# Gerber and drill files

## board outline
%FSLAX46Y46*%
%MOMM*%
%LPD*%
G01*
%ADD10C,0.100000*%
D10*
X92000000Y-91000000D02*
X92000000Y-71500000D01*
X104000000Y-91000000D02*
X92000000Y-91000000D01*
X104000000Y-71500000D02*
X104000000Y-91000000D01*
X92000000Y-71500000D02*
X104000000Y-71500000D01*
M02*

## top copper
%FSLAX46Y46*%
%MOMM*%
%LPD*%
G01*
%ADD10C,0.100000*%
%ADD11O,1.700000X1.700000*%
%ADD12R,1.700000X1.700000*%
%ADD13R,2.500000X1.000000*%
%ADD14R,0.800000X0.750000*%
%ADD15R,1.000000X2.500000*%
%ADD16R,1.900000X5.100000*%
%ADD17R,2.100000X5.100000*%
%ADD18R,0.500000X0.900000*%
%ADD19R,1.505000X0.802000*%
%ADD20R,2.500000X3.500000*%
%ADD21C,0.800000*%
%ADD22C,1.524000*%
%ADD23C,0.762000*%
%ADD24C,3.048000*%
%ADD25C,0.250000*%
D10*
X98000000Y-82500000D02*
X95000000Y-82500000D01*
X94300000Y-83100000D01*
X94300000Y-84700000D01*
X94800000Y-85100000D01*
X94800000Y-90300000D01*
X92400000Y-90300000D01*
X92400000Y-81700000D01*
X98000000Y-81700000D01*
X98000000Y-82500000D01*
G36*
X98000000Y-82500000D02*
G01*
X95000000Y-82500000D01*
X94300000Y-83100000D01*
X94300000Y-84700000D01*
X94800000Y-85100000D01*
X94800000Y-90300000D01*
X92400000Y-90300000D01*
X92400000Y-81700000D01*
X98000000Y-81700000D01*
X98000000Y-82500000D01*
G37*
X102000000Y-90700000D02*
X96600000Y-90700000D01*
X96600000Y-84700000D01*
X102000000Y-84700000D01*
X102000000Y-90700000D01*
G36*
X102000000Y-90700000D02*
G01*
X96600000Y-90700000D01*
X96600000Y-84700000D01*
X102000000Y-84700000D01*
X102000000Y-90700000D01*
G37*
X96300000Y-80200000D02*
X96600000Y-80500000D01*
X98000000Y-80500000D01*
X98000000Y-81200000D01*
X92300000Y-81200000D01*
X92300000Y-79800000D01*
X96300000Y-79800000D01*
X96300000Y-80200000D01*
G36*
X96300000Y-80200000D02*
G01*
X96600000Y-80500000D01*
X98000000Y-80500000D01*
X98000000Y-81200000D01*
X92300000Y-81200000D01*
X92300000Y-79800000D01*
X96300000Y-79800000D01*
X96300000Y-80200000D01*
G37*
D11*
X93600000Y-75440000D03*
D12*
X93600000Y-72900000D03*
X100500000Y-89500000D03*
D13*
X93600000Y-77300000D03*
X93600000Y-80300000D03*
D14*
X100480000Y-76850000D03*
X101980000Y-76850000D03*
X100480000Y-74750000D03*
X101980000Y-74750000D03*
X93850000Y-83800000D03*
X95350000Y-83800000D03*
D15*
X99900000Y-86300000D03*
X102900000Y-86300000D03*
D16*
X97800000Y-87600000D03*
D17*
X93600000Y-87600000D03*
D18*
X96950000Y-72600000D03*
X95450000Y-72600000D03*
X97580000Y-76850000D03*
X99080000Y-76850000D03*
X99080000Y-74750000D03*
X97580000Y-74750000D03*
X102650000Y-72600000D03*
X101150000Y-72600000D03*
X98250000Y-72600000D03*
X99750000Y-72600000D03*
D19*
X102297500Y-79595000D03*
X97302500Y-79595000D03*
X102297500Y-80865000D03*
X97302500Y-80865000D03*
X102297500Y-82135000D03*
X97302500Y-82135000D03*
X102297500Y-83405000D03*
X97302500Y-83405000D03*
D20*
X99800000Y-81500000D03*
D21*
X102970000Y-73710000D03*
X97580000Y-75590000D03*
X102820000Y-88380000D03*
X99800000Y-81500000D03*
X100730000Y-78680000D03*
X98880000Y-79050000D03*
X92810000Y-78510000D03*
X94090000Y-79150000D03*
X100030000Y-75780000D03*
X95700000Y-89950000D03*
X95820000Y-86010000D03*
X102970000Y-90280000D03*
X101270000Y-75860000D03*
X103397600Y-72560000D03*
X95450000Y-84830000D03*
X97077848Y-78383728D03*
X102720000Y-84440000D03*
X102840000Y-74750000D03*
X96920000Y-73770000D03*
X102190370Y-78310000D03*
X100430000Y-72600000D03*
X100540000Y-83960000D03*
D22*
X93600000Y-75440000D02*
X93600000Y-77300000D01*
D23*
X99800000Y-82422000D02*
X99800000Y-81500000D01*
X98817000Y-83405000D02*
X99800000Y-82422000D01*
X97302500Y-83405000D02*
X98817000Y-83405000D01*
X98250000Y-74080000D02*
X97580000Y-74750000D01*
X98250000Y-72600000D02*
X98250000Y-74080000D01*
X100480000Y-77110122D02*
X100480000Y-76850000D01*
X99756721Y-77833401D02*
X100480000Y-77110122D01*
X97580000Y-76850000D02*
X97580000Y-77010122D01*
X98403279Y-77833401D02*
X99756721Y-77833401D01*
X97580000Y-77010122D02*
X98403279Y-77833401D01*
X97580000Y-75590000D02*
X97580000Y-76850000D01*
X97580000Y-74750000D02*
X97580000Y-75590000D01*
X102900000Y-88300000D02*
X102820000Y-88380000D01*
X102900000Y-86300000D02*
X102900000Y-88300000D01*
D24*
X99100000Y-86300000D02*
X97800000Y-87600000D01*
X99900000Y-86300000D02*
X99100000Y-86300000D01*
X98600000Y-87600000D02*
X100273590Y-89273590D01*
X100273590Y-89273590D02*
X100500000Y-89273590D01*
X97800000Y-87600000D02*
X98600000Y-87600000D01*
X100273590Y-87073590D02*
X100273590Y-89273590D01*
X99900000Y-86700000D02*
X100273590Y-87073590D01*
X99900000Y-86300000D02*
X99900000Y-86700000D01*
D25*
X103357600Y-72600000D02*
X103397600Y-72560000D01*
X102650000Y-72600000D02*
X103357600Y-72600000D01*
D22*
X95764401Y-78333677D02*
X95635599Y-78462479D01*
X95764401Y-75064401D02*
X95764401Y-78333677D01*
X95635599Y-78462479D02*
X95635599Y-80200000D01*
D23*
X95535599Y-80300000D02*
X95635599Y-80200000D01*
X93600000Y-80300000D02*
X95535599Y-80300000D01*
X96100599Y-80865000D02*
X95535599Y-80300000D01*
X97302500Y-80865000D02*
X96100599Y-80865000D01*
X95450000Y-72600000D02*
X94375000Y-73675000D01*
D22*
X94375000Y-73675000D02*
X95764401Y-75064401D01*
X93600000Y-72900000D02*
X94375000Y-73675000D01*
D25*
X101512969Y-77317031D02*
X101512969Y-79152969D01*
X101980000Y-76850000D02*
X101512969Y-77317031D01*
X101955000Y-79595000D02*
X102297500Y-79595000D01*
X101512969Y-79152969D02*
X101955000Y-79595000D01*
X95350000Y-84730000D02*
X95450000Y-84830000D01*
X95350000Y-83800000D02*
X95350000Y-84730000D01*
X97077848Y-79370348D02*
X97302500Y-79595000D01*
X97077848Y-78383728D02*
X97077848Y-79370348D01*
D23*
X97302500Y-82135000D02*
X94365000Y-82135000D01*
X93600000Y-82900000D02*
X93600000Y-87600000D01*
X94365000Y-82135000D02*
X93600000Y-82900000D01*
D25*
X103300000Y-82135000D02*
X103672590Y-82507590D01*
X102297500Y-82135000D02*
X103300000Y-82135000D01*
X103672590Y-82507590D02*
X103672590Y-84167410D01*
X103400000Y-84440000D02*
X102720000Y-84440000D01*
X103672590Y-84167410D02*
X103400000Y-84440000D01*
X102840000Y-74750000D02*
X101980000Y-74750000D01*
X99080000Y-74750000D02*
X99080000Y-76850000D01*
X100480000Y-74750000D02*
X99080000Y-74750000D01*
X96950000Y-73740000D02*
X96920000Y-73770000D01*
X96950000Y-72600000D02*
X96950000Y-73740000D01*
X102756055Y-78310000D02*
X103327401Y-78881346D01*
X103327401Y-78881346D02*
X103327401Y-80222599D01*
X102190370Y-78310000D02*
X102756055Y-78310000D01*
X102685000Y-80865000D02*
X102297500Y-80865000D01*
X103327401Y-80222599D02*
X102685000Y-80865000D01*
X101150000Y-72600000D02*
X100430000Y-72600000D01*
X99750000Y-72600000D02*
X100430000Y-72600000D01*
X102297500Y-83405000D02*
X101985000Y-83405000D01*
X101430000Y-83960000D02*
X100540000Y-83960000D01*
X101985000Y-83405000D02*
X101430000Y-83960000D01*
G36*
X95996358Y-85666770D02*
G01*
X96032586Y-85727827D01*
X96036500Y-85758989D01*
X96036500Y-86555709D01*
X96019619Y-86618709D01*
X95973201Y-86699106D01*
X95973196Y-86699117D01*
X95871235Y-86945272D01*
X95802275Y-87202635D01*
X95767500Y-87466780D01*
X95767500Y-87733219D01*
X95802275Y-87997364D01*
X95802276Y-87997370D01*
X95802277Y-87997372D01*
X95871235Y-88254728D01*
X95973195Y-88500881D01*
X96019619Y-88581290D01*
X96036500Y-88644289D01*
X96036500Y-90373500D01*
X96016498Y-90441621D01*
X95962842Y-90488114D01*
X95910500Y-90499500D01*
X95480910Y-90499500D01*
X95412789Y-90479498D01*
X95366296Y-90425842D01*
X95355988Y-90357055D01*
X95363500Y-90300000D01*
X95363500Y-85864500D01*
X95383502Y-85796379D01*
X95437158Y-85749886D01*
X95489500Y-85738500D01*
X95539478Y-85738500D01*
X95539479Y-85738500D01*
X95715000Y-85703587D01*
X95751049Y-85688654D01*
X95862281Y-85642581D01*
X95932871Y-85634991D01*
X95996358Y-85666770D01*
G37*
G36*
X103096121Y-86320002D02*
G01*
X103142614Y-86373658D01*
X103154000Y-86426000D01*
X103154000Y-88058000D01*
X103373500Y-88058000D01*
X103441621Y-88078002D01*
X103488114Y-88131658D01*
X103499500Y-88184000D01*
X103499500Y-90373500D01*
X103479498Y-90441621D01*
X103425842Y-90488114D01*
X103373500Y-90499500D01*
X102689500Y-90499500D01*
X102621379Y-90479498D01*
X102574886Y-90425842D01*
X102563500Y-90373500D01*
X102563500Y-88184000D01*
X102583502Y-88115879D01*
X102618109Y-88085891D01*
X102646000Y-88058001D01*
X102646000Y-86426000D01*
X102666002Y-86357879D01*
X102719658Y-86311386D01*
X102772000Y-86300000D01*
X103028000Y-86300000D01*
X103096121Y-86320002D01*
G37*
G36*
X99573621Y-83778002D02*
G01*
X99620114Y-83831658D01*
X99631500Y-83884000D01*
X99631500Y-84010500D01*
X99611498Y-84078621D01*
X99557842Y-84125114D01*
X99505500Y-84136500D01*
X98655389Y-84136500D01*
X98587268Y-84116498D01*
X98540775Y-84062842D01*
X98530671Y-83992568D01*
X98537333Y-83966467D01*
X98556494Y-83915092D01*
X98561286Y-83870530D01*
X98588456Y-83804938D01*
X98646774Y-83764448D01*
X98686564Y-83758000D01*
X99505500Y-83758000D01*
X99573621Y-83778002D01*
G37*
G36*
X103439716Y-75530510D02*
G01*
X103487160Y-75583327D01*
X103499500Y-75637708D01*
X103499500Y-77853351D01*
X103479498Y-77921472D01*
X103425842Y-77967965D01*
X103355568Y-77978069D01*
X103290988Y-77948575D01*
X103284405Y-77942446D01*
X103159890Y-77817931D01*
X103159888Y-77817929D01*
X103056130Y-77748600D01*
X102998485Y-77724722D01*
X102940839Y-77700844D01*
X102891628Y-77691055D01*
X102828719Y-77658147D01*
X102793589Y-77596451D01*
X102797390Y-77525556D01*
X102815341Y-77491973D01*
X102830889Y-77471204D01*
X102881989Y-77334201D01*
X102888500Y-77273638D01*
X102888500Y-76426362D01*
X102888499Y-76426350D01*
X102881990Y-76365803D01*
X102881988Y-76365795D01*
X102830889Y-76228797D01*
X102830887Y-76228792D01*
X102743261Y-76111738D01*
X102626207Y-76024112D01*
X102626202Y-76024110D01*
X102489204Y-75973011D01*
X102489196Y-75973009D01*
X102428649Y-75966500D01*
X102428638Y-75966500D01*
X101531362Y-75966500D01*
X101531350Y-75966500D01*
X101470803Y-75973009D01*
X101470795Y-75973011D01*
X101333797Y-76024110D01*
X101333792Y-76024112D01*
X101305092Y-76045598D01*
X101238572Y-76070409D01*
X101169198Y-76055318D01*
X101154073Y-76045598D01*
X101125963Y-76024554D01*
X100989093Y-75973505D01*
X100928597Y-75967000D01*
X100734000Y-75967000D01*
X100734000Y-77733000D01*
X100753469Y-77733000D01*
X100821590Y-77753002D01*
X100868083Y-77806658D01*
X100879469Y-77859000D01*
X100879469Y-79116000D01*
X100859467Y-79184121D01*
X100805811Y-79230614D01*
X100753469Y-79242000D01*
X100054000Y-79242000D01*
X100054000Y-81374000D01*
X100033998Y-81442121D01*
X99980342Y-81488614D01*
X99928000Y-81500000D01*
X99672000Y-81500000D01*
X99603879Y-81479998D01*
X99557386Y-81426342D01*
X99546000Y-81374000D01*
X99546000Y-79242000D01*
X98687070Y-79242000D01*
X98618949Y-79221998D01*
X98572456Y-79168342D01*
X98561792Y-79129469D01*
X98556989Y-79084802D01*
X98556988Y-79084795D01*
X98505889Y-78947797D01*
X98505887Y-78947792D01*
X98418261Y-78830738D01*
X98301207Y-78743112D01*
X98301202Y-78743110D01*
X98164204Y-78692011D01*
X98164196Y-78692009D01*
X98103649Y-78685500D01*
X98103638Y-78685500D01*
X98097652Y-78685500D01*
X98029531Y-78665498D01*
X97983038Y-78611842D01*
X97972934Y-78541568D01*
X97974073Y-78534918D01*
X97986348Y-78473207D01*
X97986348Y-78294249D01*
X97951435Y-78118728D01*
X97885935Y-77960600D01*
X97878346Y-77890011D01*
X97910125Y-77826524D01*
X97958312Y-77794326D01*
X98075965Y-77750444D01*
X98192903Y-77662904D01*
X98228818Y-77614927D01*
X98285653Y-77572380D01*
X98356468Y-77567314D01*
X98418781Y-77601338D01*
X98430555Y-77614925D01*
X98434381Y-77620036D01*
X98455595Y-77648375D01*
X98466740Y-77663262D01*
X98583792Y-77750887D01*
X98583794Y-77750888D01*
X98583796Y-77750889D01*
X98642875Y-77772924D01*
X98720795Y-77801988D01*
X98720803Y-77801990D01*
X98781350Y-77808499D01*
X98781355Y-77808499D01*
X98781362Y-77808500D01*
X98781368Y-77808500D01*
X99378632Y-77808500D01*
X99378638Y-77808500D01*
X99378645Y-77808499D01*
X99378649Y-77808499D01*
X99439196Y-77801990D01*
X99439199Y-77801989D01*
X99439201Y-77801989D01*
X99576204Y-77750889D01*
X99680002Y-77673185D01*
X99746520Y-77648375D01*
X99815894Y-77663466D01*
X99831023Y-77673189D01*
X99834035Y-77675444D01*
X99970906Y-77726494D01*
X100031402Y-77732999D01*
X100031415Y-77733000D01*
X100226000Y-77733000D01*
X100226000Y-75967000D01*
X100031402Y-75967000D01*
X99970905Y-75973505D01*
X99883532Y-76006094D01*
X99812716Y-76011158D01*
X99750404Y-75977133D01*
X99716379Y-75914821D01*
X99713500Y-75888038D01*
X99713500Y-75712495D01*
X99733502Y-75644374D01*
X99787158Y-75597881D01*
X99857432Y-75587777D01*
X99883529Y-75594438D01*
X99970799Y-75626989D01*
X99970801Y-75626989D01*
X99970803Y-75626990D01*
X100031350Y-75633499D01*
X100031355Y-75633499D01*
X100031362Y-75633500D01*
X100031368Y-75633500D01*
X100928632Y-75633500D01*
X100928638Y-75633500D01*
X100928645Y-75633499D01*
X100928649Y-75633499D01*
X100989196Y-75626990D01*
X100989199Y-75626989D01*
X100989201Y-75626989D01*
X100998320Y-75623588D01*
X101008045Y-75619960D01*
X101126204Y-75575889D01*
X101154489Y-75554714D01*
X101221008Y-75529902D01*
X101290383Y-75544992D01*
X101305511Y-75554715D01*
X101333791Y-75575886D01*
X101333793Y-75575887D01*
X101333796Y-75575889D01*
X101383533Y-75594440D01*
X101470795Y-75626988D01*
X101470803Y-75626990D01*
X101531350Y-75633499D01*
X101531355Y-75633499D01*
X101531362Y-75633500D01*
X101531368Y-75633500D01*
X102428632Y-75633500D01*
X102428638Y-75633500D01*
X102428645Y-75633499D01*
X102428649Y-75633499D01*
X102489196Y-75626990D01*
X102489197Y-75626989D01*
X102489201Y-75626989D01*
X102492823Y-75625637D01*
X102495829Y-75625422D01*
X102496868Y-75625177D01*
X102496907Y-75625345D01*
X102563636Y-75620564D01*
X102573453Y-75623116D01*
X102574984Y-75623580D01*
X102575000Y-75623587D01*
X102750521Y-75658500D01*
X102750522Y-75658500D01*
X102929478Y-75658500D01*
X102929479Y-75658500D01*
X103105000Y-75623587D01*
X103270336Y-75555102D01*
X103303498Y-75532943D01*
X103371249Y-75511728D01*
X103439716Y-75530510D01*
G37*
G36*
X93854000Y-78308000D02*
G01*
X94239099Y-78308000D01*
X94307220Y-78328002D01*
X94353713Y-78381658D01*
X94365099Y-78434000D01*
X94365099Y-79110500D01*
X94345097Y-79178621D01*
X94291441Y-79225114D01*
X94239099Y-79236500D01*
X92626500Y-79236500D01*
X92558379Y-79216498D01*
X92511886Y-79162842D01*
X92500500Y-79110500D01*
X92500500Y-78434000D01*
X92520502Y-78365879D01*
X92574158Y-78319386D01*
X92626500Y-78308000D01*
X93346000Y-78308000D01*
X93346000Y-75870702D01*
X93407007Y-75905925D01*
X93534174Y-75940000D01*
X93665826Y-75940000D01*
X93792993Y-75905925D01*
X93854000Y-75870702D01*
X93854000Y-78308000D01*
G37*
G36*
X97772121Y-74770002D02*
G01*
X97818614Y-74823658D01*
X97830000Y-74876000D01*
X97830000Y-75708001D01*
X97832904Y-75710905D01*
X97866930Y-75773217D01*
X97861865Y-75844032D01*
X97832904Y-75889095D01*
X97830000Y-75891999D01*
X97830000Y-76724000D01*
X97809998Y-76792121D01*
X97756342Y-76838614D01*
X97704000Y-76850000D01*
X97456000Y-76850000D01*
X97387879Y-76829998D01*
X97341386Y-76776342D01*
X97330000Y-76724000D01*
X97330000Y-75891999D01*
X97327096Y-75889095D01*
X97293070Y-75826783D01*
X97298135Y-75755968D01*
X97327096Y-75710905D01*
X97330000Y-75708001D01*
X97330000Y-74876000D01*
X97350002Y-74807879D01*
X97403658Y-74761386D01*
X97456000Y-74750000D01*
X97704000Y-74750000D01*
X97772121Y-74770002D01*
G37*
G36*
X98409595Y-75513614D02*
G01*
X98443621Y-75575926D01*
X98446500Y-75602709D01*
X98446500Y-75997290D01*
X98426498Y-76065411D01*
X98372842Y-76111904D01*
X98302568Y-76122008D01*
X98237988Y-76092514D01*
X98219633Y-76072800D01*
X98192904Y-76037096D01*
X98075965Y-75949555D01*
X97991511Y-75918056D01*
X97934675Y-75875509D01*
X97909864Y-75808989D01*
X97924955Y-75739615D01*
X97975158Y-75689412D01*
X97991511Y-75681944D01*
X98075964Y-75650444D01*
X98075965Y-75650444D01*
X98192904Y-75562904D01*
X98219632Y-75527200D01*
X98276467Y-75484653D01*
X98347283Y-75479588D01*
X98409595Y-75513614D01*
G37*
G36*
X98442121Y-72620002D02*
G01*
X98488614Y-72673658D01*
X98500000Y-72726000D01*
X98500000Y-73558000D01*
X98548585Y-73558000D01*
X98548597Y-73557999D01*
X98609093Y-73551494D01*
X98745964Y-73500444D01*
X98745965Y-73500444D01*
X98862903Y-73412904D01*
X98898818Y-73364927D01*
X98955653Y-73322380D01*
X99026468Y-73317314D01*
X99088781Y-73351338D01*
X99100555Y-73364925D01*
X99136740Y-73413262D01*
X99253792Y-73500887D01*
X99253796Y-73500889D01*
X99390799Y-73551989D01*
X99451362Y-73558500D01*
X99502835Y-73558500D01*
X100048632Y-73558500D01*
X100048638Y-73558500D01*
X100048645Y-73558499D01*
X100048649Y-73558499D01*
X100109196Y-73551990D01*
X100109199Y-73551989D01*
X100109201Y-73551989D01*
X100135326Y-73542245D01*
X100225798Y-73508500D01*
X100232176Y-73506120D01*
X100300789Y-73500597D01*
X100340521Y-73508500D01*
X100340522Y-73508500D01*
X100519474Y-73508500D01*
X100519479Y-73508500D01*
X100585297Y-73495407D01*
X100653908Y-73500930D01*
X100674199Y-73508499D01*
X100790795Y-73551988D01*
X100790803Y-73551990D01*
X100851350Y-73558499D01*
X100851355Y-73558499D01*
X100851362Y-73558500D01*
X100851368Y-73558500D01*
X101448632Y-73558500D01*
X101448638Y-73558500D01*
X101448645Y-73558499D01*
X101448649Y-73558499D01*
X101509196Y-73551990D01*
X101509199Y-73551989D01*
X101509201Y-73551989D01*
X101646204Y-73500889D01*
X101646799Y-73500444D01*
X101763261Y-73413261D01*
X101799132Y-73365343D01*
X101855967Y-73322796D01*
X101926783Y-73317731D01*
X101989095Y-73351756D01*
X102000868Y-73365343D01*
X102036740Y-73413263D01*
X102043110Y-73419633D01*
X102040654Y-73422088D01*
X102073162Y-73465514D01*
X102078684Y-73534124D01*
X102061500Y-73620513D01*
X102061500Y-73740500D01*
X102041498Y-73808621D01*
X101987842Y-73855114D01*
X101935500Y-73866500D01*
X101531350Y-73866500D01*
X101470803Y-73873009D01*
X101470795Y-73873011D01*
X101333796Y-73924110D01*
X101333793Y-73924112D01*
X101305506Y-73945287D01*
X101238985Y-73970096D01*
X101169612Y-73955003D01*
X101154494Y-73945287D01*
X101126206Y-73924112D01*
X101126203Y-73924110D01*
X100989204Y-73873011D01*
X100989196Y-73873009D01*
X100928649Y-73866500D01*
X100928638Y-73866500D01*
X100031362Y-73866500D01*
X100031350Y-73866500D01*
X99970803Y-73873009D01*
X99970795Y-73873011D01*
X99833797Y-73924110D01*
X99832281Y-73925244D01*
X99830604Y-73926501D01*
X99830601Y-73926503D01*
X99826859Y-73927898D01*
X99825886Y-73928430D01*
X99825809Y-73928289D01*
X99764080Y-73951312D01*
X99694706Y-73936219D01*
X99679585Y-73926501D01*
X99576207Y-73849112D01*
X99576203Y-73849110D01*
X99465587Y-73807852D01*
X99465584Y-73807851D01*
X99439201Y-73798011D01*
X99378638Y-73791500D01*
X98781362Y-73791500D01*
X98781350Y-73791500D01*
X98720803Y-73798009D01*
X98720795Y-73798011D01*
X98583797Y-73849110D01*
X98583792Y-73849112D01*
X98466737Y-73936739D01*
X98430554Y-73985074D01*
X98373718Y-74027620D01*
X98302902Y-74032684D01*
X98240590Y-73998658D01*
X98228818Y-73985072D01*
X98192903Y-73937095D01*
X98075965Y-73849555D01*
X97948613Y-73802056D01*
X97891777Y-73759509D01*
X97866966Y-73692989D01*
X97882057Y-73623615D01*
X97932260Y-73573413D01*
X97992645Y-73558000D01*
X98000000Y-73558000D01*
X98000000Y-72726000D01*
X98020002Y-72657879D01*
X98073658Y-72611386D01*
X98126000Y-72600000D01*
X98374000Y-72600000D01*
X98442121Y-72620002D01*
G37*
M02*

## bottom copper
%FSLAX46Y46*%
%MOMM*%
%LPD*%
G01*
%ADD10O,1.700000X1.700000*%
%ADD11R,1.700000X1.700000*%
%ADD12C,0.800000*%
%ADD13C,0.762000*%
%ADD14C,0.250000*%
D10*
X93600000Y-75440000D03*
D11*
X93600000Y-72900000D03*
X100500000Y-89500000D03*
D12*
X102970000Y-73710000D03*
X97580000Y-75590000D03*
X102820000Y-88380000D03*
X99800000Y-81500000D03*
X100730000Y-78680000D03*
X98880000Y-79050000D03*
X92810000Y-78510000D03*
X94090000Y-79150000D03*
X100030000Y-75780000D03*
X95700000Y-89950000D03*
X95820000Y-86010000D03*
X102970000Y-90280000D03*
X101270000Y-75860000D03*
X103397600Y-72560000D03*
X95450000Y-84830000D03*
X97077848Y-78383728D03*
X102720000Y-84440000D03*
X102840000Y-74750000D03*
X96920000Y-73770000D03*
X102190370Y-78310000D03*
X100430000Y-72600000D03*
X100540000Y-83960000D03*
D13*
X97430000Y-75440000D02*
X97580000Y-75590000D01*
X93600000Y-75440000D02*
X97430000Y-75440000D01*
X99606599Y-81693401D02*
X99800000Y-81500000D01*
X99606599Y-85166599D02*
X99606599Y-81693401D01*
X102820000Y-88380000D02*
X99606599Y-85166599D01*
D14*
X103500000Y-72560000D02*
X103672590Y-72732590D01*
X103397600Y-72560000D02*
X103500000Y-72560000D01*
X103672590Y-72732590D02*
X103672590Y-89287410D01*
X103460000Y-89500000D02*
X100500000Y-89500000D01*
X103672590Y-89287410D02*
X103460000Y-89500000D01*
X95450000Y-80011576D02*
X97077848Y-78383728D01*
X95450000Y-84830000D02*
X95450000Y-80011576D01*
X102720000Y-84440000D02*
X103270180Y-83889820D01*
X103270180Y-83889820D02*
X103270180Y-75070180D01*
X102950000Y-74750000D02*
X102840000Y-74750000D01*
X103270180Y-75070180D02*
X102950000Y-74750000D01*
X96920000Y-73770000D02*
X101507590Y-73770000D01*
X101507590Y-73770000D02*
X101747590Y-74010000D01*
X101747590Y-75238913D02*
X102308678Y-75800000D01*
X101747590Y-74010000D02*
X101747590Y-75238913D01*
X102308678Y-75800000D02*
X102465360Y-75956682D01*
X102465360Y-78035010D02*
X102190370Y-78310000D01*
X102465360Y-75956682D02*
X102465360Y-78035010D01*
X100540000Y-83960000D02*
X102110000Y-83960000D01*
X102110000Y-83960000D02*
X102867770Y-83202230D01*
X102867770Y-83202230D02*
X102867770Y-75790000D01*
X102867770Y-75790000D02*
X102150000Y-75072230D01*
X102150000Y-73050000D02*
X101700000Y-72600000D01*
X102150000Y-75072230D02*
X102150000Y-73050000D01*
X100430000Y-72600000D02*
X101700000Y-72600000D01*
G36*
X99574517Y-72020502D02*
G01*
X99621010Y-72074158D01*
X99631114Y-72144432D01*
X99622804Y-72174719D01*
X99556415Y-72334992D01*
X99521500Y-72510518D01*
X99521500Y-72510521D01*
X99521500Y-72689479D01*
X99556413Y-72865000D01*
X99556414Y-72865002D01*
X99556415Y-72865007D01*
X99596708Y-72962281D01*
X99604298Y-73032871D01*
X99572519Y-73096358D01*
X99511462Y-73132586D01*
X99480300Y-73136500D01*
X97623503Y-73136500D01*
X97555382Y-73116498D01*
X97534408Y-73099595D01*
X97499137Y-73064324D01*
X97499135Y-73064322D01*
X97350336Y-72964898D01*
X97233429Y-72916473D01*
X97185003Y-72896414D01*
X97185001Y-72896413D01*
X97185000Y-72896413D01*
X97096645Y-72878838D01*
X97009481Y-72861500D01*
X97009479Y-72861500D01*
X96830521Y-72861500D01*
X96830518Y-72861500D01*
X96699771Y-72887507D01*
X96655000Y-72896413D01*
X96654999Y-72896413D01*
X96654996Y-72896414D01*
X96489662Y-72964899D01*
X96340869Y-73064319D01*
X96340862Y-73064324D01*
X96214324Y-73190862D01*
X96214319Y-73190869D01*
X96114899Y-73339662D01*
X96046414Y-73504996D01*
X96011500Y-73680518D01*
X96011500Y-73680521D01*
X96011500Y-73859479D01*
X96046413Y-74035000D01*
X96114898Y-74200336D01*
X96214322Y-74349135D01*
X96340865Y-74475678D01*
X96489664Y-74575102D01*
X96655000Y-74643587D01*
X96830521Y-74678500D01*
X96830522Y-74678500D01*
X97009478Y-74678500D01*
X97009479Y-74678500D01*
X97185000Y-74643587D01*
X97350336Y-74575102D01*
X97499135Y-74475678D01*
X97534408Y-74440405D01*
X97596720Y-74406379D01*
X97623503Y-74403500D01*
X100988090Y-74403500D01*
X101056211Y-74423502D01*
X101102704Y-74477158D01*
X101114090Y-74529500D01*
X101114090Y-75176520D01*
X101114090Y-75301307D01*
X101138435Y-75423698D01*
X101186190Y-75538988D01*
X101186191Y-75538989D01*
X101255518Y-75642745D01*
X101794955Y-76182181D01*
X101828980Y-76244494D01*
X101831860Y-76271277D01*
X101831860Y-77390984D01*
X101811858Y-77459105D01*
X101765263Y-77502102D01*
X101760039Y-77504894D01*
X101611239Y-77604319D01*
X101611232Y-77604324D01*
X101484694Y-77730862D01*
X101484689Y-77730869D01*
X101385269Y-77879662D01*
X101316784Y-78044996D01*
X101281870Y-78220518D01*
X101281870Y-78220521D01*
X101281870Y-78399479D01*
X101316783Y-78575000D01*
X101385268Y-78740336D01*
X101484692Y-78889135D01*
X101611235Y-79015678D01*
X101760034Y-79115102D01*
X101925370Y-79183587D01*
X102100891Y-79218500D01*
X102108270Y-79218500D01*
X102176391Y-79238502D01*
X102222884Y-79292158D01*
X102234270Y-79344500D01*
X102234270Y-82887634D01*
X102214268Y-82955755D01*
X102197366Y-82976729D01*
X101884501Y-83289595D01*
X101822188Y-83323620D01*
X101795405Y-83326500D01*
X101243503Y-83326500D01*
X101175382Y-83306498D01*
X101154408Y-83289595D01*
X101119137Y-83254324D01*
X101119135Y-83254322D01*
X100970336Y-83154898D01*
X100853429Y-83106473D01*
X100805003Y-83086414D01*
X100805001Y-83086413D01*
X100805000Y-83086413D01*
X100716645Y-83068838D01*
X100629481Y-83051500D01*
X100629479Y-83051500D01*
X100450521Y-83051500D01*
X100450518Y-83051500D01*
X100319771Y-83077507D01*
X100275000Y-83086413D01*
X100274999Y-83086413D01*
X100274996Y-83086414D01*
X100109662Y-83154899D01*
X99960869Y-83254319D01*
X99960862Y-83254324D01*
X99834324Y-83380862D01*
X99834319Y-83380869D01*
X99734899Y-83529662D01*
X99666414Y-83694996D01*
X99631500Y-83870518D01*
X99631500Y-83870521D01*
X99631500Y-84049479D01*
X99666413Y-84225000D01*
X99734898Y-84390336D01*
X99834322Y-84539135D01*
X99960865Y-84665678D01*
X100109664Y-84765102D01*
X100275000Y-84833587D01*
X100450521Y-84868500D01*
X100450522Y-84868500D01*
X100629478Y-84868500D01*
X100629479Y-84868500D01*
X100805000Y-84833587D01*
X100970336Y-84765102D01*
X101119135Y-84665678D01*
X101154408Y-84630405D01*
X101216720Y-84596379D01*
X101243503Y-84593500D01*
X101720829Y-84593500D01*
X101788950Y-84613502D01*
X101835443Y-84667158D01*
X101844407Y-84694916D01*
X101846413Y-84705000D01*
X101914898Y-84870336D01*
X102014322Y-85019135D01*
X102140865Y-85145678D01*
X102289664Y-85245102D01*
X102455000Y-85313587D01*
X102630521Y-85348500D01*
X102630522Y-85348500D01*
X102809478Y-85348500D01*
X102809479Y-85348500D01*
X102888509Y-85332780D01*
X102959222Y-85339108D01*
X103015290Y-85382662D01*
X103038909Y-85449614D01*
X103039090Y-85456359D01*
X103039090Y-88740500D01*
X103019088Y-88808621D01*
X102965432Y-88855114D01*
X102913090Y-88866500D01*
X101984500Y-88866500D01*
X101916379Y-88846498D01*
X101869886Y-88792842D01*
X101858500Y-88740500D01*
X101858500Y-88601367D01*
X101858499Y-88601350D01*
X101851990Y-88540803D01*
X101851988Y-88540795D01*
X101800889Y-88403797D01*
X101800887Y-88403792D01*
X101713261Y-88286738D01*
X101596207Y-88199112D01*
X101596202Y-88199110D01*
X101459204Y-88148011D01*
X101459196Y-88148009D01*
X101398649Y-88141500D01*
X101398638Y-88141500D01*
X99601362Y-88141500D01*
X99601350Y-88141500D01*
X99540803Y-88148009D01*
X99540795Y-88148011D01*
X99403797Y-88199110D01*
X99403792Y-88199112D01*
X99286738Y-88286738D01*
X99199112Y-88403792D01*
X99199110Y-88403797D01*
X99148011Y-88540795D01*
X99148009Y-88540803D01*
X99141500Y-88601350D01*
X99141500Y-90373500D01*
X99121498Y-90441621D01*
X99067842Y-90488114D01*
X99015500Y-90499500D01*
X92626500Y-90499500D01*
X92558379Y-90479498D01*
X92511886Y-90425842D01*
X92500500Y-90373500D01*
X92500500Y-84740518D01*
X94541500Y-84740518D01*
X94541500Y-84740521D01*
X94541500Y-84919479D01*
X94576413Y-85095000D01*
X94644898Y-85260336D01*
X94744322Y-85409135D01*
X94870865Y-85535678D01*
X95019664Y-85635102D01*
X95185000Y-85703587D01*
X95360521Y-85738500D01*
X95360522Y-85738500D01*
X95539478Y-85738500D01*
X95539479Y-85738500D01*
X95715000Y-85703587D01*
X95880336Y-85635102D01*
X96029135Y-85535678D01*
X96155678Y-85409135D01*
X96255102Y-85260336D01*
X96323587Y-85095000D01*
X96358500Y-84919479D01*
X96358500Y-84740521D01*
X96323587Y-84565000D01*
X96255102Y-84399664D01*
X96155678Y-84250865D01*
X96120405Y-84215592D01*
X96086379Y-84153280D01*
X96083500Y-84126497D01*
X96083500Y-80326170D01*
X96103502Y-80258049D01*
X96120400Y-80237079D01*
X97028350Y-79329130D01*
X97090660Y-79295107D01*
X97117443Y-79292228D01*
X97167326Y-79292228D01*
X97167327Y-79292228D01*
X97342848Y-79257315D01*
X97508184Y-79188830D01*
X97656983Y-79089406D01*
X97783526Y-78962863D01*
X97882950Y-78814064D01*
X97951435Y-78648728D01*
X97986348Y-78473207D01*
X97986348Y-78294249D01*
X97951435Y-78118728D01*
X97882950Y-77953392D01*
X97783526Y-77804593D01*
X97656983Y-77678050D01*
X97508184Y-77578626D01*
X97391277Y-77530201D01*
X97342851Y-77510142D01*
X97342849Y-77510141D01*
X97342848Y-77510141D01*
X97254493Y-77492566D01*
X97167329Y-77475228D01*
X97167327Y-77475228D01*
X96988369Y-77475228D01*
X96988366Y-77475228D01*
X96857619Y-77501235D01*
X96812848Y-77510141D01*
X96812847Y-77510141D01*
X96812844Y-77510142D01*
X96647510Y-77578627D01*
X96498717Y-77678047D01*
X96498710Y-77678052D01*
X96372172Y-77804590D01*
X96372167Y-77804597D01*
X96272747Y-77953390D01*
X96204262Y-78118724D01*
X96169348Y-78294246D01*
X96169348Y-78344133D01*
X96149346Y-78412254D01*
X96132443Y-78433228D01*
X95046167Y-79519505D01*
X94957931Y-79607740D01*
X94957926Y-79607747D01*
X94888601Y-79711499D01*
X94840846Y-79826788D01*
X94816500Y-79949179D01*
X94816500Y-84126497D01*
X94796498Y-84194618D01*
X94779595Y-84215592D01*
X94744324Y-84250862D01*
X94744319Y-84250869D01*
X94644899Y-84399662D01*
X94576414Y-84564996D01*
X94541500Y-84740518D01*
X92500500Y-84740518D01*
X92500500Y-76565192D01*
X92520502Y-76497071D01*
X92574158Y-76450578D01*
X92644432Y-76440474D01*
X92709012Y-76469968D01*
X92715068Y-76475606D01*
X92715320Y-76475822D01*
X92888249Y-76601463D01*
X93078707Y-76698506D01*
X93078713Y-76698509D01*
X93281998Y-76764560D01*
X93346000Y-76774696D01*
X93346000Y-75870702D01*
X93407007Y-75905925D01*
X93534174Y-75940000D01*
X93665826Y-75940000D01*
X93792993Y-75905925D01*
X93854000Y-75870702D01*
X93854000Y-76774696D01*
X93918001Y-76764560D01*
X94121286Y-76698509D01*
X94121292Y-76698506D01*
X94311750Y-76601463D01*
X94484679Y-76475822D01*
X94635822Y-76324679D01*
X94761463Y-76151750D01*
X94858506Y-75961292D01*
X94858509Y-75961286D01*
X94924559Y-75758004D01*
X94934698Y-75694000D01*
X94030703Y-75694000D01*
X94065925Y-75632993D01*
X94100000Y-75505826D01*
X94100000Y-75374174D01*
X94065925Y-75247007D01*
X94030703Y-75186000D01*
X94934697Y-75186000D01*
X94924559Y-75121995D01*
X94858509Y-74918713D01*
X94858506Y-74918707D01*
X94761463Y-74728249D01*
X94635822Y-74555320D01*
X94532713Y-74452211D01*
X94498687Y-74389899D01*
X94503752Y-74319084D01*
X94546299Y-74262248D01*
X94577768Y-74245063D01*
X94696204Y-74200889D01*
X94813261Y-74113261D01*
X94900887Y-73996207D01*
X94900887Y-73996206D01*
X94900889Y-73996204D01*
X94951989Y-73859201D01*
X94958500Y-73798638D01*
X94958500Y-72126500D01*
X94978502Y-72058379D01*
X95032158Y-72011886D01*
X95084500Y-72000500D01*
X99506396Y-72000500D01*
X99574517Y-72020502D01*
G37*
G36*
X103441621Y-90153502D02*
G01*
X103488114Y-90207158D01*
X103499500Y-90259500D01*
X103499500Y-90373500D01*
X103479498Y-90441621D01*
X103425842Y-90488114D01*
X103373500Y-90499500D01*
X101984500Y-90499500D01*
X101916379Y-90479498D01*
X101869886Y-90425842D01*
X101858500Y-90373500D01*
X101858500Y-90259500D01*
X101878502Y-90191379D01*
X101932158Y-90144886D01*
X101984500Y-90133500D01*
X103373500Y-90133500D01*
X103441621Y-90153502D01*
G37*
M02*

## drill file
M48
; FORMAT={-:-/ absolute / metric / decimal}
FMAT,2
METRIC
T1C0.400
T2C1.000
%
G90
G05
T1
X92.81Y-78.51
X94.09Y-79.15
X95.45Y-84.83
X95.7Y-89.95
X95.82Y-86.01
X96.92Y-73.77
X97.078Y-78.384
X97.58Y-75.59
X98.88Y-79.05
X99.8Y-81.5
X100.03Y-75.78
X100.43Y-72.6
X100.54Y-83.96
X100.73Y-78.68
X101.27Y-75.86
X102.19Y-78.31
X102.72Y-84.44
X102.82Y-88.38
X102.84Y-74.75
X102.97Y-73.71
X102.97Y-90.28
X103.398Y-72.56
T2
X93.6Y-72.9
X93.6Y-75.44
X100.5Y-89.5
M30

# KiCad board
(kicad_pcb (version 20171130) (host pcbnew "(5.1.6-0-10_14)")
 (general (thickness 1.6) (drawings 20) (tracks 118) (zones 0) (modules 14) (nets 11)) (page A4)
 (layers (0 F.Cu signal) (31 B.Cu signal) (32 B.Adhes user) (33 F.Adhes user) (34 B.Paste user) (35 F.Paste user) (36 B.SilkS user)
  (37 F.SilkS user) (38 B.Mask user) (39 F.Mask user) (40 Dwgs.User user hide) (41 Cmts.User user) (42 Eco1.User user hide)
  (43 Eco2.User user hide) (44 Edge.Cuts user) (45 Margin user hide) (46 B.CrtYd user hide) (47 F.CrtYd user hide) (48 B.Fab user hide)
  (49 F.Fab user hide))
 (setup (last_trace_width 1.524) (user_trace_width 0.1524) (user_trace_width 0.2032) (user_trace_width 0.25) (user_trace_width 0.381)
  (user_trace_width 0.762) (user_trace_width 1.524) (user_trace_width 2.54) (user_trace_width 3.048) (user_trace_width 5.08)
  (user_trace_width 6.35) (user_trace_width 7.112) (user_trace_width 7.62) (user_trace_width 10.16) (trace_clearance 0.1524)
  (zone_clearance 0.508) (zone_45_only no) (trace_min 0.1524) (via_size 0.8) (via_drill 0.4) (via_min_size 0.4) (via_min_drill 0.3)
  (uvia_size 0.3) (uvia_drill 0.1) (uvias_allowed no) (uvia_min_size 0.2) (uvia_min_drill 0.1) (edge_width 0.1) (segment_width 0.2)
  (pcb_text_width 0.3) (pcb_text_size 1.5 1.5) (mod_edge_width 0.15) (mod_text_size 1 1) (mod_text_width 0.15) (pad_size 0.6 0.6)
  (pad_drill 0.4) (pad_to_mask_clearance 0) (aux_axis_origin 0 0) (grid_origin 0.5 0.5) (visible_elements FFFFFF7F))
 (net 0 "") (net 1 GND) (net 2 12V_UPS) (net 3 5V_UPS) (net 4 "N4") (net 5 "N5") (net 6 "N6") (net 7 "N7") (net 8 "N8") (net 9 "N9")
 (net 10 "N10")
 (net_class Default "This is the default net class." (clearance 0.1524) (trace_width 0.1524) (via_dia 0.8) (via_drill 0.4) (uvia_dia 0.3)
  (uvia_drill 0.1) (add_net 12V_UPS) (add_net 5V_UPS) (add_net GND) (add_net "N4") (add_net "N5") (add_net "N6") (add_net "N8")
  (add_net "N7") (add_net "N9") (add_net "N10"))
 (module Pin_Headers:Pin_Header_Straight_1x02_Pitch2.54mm (layer F.Cu) (at 93.6 72.9)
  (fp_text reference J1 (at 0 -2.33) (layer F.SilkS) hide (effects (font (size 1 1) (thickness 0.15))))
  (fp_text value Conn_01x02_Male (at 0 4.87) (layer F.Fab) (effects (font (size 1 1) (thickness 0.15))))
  (pad 2 thru_hole oval (at 0 2.54) (size 1.7 1.7) (drill 1) (layers *.Cu *.Mask) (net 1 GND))
  (pad 1 thru_hole rect (at 0 0) (size 1.7 1.7) (drill 1) (layers *.Cu *.Mask) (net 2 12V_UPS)))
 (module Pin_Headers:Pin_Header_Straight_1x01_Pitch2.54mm (layer F.Cu) (at 100.5 89.5)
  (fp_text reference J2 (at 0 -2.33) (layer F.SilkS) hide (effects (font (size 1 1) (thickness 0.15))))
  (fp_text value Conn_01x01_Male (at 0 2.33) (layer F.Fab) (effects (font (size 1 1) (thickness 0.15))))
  (pad 1 thru_hole rect (at 0 0) (size 1.7 1.7) (drill 1) (layers *.Cu *.Mask) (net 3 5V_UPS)))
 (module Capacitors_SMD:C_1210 (layer F.Cu) (at 93.6 78.8 270)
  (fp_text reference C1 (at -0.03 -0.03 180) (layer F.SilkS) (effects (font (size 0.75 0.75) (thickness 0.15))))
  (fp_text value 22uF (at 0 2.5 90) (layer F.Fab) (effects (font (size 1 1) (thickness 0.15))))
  (pad 1 smd rect (at -1.5 0 270) (size 1 2.5) (layers F.Cu F.Paste F.Mask) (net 1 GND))
  (pad 2 smd rect (at 1.5 0 270) (size 1 2.5) (layers F.Cu F.Paste F.Mask) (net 2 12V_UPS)))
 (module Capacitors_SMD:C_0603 (layer F.Cu) (at 101.23 76.85)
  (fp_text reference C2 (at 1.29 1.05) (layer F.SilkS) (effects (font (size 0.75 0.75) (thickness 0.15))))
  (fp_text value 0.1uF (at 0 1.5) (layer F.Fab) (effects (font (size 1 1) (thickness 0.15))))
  (pad 1 smd rect (at -0.75 0) (size 0.8 0.75) (layers F.Cu F.Paste F.Mask) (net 1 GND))
  (pad 2 smd rect (at 0.75 0) (size 0.8 0.75) (layers F.Cu F.Paste F.Mask) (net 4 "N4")))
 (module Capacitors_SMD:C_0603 (layer F.Cu) (at 101.23 74.75)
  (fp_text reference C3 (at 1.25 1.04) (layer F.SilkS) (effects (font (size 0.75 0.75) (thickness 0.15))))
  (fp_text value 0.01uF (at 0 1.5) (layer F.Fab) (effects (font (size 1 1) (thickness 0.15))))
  (pad 1 smd rect (at -0.75 0) (size 0.8 0.75) (layers F.Cu F.Paste F.Mask) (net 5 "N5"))
  (pad 2 smd rect (at 0.75 0) (size 0.8 0.75) (layers F.Cu F.Paste F.Mask) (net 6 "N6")))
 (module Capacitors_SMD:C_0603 (layer F.Cu) (at 94.6 83.8 180)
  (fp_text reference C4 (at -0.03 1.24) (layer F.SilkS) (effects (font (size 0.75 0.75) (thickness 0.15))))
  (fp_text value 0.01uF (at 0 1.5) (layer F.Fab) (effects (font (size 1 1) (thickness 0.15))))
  (pad 2 smd rect (at 0.75 0 180) (size 0.8 0.75) (layers F.Cu F.Paste F.Mask) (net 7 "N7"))
  (pad 1 smd rect (at -0.75 0 180) (size 0.8 0.75) (layers F.Cu F.Paste F.Mask) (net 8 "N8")))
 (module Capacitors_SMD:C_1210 (layer F.Cu) (at 101.4 86.3 180)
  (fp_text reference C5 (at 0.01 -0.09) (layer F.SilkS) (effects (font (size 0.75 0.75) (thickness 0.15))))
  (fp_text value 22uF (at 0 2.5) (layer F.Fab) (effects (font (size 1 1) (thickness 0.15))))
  (pad 2 smd rect (at 1.5 0 180) (size 1 2.5) (layers F.Cu F.Paste F.Mask) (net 3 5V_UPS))
  (pad 1 smd rect (at -1.5 0 180) (size 1 2.5) (layers F.Cu F.Paste F.Mask) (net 1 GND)))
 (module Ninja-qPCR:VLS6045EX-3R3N (layer F.Cu) (at 95.7 87.6 180)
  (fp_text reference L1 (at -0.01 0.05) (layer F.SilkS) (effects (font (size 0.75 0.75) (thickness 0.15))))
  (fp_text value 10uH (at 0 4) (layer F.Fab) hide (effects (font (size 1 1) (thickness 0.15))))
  (pad 1 smd rect (at -2.1 0 180) (size 1.9 5.1) (layers F.Cu F.Paste F.Mask) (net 3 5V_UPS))
  (pad 2 smd rect (at 2.1 0 180) (size 2.1 5.1) (layers F.Cu F.Paste F.Mask) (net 7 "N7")))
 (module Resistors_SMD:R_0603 (layer F.Cu) (at 96.2 72.6)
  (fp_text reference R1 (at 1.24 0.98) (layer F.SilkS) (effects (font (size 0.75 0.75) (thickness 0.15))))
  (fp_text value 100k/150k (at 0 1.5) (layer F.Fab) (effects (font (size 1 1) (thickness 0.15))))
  (pad 2 smd rect (at 0.75 0) (size 0.5 0.9) (layers F.Cu F.Paste F.Mask) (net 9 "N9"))
  (pad 1 smd rect (at -0.75 0) (size 0.5 0.9) (layers F.Cu F.Paste F.Mask) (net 2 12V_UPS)))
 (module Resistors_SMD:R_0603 (layer F.Cu) (at 98.33 76.85 180)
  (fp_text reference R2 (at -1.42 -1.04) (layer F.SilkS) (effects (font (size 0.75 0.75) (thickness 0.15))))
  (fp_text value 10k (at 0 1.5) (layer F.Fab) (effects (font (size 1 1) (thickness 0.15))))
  (pad 2 smd rect (at 0.75 0 180) (size 0.5 0.9) (layers F.Cu F.Paste F.Mask) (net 1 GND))
  (pad 1 smd rect (at -0.75 0 180) (size 0.5 0.9) (layers F.Cu F.Paste F.Mask) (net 5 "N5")))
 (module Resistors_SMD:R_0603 (layer F.Cu) (at 98.33 74.75 180)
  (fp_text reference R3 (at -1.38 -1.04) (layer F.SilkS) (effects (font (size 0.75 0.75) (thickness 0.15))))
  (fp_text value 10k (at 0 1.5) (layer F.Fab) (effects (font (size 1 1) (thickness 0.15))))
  (pad 1 smd rect (at -0.75 0 180) (size 0.5 0.9) (layers F.Cu F.Paste F.Mask) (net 5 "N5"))
  (pad 2 smd rect (at 0.75 0 180) (size 0.5 0.9) (layers F.Cu F.Paste F.Mask) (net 1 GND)))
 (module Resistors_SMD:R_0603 (layer F.Cu) (at 101.9 72.6 180)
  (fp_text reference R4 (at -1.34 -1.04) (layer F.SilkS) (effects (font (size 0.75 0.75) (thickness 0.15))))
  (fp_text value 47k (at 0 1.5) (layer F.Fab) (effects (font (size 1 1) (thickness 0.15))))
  (pad 1 smd rect (at -0.75 0 180) (size 0.5 0.9) (layers F.Cu F.Paste F.Mask) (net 3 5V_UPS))
  (pad 2 smd rect (at 0.75 0 180) (size 0.5 0.9) (layers F.Cu F.Paste F.Mask) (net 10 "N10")))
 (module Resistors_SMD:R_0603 (layer F.Cu) (at 99 72.6 180)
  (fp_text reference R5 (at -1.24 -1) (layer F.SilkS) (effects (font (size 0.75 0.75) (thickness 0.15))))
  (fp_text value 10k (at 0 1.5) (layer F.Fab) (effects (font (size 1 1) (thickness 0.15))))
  (pad 2 smd rect (at 0.75 0 180) (size 0.5 0.9) (layers F.Cu F.Paste F.Mask) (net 1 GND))
  (pad 1 smd rect (at -0.75 0 180) (size 0.5 0.9) (layers F.Cu F.Paste F.Mask) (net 10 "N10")))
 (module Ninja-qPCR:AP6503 (layer F.Cu) (at 99.8 81.5 270)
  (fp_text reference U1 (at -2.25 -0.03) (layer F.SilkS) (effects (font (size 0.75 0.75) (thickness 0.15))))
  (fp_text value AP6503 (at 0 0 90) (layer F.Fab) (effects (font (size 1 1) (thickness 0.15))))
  (pad 8 smd rect (at -1.905 -2.4975 270) (size 0.802 1.505) (layers F.Cu F.Paste F.Mask) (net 4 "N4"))
  (pad 1 smd rect (at -1.905 2.4975 270) (size 0.802 1.505) (layers F.Cu F.Paste F.Mask) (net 8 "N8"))
  (pad 7 smd rect (at -0.635 -2.4975 270) (size 0.802 1.505) (layers F.Cu F.Paste F.Mask) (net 9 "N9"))
  (pad 2 smd rect (at -0.635 2.4975 270) (size 0.802 1.505) (layers F.Cu F.Paste F.Mask) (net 2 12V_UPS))
  (pad 6 smd rect (at 0.635 -2.4975 270) (size 0.802 1.505) (layers F.Cu F.Paste F.Mask) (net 6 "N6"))
  (pad 3 smd rect (at 0.635 2.4975 270) (size 0.802 1.505) (layers F.Cu F.Paste F.Mask) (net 7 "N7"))
  (pad 5 smd rect (at 1.905 -2.4975 270) (size 0.802 1.505) (layers F.Cu F.Paste F.Mask) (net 10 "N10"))
  (pad 4 smd rect (at 1.905 2.4975 270) (size 0.802 1.505) (layers F.Cu F.Paste F.Mask) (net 1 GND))
  (pad 9 smd rect (at 0 0 270) (size 3.5 2.5) (layers F.Cu F.Paste F.Mask) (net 1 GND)))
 (gr_poly
  (pts (xy 98 82.5) (xy 95 82.5) (xy 94.3 83.1) (xy 94.3 84.7) (xy 94.8 85.1) (xy 94.8 90.3) (xy 92.4 90.3) (xy 92.4 81.7) (xy 98 81.7))
  (layer F.Cu) (width 0.1))
 (gr_poly (pts (xy 102 90.7) (xy 96.6 90.7) (xy 96.6 84.7) (xy 102 84.7)) (layer F.Cu) (width 0.1))
 (gr_poly
  (pts (xy 96.3 80.2) (xy 96.6 80.5) (xy 98 80.5) (xy 98 81.2) (xy 92.3 81.2) (xy 92.3 79.8) (xy 96.3 79.8)) (layer F.Cu) (width 0.1))
 (gr_line (start 92 91) (end 92 71.5) (layer Edge.Cuts) (width 0.1))
 (gr_line (start 104 91) (end 92 91) (layer Edge.Cuts) (width 0.1))
 (gr_line (start 104 71.5) (end 104 91) (layer Edge.Cuts) (width 0.1))
 (gr_line (start 92 71.5) (end 104 71.5) (layer Edge.Cuts) (width 0.1))
 (via (at 102.97 73.71) (size 0.8) (drill 0.4) (layers F.Cu B.Cu) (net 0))
 (segment (start 93.6 75.44) (end 93.6 77.3) (width 1.524) (layer F.Cu) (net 1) (status 30))
 (segment (start 99.8 82.422) (end 99.8 81.5) (width 0.762) (layer F.Cu) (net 1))
 (segment (start 98.817 83.405) (end 99.8 82.422) (width 0.762) (layer F.Cu) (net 1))
 (segment (start 97.3025 83.405) (end 98.817 83.405) (width 0.762) (layer F.Cu) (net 1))
 (segment (start 98.25 74.08) (end 97.58 74.75) (width 0.762) (layer F.Cu) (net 1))
 (segment (start 98.25 72.6) (end 98.25 74.08) (width 0.762) (layer F.Cu) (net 1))
 (segment (start 100.48 77.110122) (end 100.48 76.85) (width 0.762) (layer F.Cu) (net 1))
 (segment (start 99.756721 77.833401) (end 100.48 77.110122) (width 0.762) (layer F.Cu) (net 1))
 (segment (start 97.58 76.85) (end 97.58 77.010122) (width 0.762) (layer F.Cu) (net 1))
 (segment (start 98.403279 77.833401) (end 99.756721 77.833401) (width 0.762) (layer F.Cu) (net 1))
 (segment (start 97.58 77.010122) (end 98.403279 77.833401) (width 0.762) (layer F.Cu) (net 1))
 (via (at 97.58 75.59) (size 0.8) (drill 0.4) (layers F.Cu B.Cu) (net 1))
 (segment (start 97.43 75.44) (end 97.58 75.59) (width 0.762) (layer B.Cu) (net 1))
 (segment (start 93.6 75.44) (end 97.43 75.44) (width 0.762) (layer B.Cu) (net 1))
 (segment (start 97.58 75.59) (end 97.58 76.85) (width 0.762) (layer F.Cu) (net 1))
 (segment (start 97.58 74.75) (end 97.58 75.59) (width 0.762) (layer F.Cu) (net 1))
 (segment (start 102.9 88.3) (end 102.82 88.38) (width 0.762) (layer F.Cu) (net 1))
 (via (at 102.82 88.38) (size 0.8) (drill 0.4) (layers F.Cu B.Cu) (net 1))
 (segment (start 102.9 86.3) (end 102.9 88.3) (width 0.762) (layer F.Cu) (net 1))
 (via (at 99.8 81.5) (size 0.8) (drill 0.4) (layers F.Cu B.Cu) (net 1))
 (segment (start 99.606599 81.693401) (end 99.8 81.5) (width 0.762) (layer B.Cu) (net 1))
 (segment (start 99.606599 85.166599) (end 99.606599 81.693401) (width 0.762) (layer B.Cu) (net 1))
 (segment (start 102.82 88.38) (end 99.606599 85.166599) (width 0.762) (layer B.Cu) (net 1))
 (via (at 100.73 78.68) (size 0.8) (drill 0.4) (layers F.Cu B.Cu) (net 1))
 (via (at 98.88 79.05) (size 0.8) (drill 0.4) (layers F.Cu B.Cu) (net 1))
 (via (at 92.81 78.51) (size 0.8) (drill 0.4) (layers F.Cu B.Cu) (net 1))
 (via (at 94.09 79.15) (size 0.8) (drill 0.4) (layers F.Cu B.Cu) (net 1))
 (via (at 100.03 75.78) (size 0.8) (drill 0.4) (layers F.Cu B.Cu) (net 1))
 (via (at 95.7 89.95) (size 0.8) (drill 0.4) (layers F.Cu B.Cu) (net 1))
 (via (at 95.82 86.01) (size 0.8) (drill 0.4) (layers F.Cu B.Cu) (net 1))
 (via (at 102.97 90.28) (size 0.8) (drill 0.4) (layers F.Cu B.Cu) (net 1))
 (via (at 101.27 75.86) (size 0.8) (drill 0.4) (layers F.Cu B.Cu) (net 1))
 (segment (start 99.1 86.3) (end 97.8 87.6) (width 3.048) (layer F.Cu) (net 3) (status 20))
 (segment (start 99.9 86.3) (end 99.1 86.3) (width 3.048) (layer F.Cu) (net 3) (status 10))
 (segment (start 98.6 87.6) (end 100.27359 89.27359) (width 3.048) (layer F.Cu) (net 3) (status 30))
 (segment (start 100.27359 89.27359) (end 100.5 89.27359) (width 3.048) (layer F.Cu) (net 3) (status 30))
 (segment (start 97.8 87.6) (end 98.6 87.6) (width 3.048) (layer F.Cu) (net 3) (status 30))
 (segment (start 100.27359 87.07359) (end 100.27359 89.27359) (width 3.048) (layer F.Cu) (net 3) (status 30))
 (segment (start 99.9 86.7) (end 100.27359 87.07359) (width 3.048) (layer F.Cu) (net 3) (status 30))
 (segment (start 99.9 86.3) (end 99.9 86.7) (width 3.048) (layer F.Cu) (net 3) (status 30))
 (via (at 103.3976 72.56) (size 0.8) (drill 0.4) (layers F.Cu B.Cu) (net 3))
 (segment (start 103.3576 72.6) (end 103.3976 72.56) (width 0.25) (layer F.Cu) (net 3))
 (segment (start 102.65 72.6) (end 103.3576 72.6) (width 0.25) (layer F.Cu) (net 3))
 (segment (start 103.5 72.56) (end 103.67259 72.73259) (width 0.25) (layer B.Cu) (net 3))
 (segment (start 103.3976 72.56) (end 103.5 72.56) (width 0.25) (layer B.Cu) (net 3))
 (segment (start 103.67259 72.73259) (end 103.67259 89.28741) (width 0.25) (layer B.Cu) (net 3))
 (segment (start 103.46 89.5) (end 100.5 89.5) (width 0.25) (layer B.Cu) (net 3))
 (segment (start 103.67259 89.28741) (end 103.46 89.5) (width 0.25) (layer B.Cu) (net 3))
 (segment (start 95.764401 78.333677) (end 95.635599 78.462479) (width 1.524) (layer F.Cu) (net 2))
 (segment (start 95.764401 75.064401) (end 95.764401 78.333677) (width 1.524) (layer F.Cu) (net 2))
 (segment (start 95.635599 78.462479) (end 95.635599 80.2) (width 1.524) (layer F.Cu) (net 2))
 (segment (start 95.535599 80.3) (end 95.635599 80.2) (width 0.762) (layer F.Cu) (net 2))
 (segment (start 93.6 80.3) (end 95.535599 80.3) (width 0.762) (layer F.Cu) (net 2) (status 10))
 (segment (start 96.100599 80.865) (end 95.535599 80.3) (width 0.762) (layer F.Cu) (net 2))
 (segment (start 97.3025 80.865) (end 96.100599 80.865) (width 0.762) (layer F.Cu) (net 2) (status 10))
 (segment (start 95.45 72.6) (end 94.375 73.675) (width 0.762) (layer F.Cu) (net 2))
 (segment (start 94.375 73.675) (end 95.764401 75.064401) (width 1.524) (layer F.Cu) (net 2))
 (segment (start 93.6 72.9) (end 94.375 73.675) (width 1.524) (layer F.Cu) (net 2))
 (segment (start 101.512969 77.317031) (end 101.512969 79.152969) (width 0.25) (layer F.Cu) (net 4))
 (segment (start 101.98 76.85) (end 101.512969 77.317031) (width 0.25) (layer F.Cu) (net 4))
 (segment (start 101.955 79.595) (end 102.2975 79.595) (width 0.25) (layer F.Cu) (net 4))
 (segment (start 101.512969 79.152969) (end 101.955 79.595) (width 0.25) (layer F.Cu) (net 4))
 (via (at 95.45 84.83) (size 0.8) (drill 0.4) (layers F.Cu B.Cu) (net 8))
 (segment (start 95.35 84.73) (end 95.45 84.83) (width 0.25) (layer F.Cu) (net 8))
 (segment (start 95.35 83.8) (end 95.35 84.73) (width 0.25) (layer F.Cu) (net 8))
 (via (at 97.077848 78.383728) (size 0.8) (drill 0.4) (layers F.Cu B.Cu) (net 8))
 (segment (start 95.45 80.011576) (end 97.077848 78.383728) (width 0.25) (layer B.Cu) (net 8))
 (segment (start 95.45 84.83) (end 95.45 80.011576) (width 0.25) (layer B.Cu) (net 8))
 (segment (start 97.077848 79.370348) (end 97.3025 79.595) (width 0.25) (layer F.Cu) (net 8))
 (segment (start 97.077848 78.383728) (end 97.077848 79.370348) (width 0.25) (layer F.Cu) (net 8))
 (segment (start 97.3025 82.135) (end 94.365 82.135) (width 0.762) (layer F.Cu) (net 7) (status 10))
 (segment (start 93.6 82.9) (end 93.6 87.6) (width 0.762) (layer F.Cu) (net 7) (status 20))
 (segment (start 94.365 82.135) (end 93.6 82.9) (width 0.762) (layer F.Cu) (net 7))
 (segment (start 103.3 82.135) (end 103.67259 82.50759) (width 0.25) (layer F.Cu) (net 6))
 (segment (start 102.2975 82.135) (end 103.3 82.135) (width 0.25) (layer F.Cu) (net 6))
 (segment (start 103.67259 82.50759) (end 103.67259 84.16741) (width 0.25) (layer F.Cu) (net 6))
 (via (at 102.72 84.44) (size 0.8) (drill 0.4) (layers F.Cu B.Cu) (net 6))
 (segment (start 103.4 84.44) (end 102.72 84.44) (width 0.25) (layer F.Cu) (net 6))
 (segment (start 103.67259 84.16741) (end 103.4 84.44) (width 0.25) (layer F.Cu) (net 6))
 (segment (start 102.72 84.44) (end 103.27018 83.88982) (width 0.25) (layer B.Cu) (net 6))
 (segment (start 103.27018 83.88982) (end 103.27018 75.07018) (width 0.25) (layer B.Cu) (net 6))
 (via (at 102.84 74.75) (size 0.8) (drill 0.4) (layers F.Cu B.Cu) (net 6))
 (segment (start 102.95 74.75) (end 102.84 74.75) (width 0.25) (layer B.Cu) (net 6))
 (segment (start 103.27018 75.07018) (end 102.95 74.75) (width 0.25) (layer B.Cu) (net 6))
 (segment (start 102.84 74.75) (end 101.98 74.75) (width 0.25) (layer F.Cu) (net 6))
 (segment (start 99.08 74.75) (end 99.08 76.85) (width 0.25) (layer F.Cu) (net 5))
 (segment (start 100.48 74.75) (end 99.08 74.75) (width 0.25) (layer F.Cu) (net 5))
 (via (at 96.92 73.77) (size 0.8) (drill 0.4) (layers F.Cu B.Cu) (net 9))
 (segment (start 96.95 73.74) (end 96.92 73.77) (width 0.25) (layer F.Cu) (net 9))
 (segment (start 96.95 72.6) (end 96.95 73.74) (width 0.25) (layer F.Cu) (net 9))
 (segment (start 96.92 73.77) (end 101.50759 73.77) (width 0.25) (layer B.Cu) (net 9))
 (segment (start 101.50759 73.77) (end 101.74759 74.01) (width 0.25) (layer B.Cu) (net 9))
 (segment (start 101.74759 75.238913) (end 102.308678 75.8) (width 0.25) (layer B.Cu) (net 9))
 (segment (start 101.74759 74.01) (end 101.74759 75.238913) (width 0.25) (layer B.Cu) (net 9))
 (segment (start 102.308678 75.8) (end 102.46536 75.956682) (width 0.25) (layer B.Cu) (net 9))
 (via (at 102.19037 78.31) (size 0.8) (drill 0.4) (layers F.Cu B.Cu) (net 9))
 (segment (start 102.46536 78.03501) (end 102.19037 78.31) (width 0.25) (layer B.Cu) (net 9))
 (segment (start 102.46536 75.956682) (end 102.46536 78.03501) (width 0.25) (layer B.Cu) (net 9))
 (segment (start 102.756055 78.31) (end 103.327401 78.881346) (width 0.25) (layer F.Cu) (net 9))
 (segment (start 103.327401 78.881346) (end 103.327401 80.222599) (width 0.25) (layer F.Cu) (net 9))
 (segment (start 102.19037 78.31) (end 102.756055 78.31) (width 0.25) (layer F.Cu) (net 9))
 (segment (start 102.685 80.865) (end 102.2975 80.865) (width 0.25) (layer F.Cu) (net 9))
 (segment (start 103.327401 80.222599) (end 102.685 80.865) (width 0.25) (layer F.Cu) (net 9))
 (via (at 100.43 72.6) (size 0.8) (drill 0.4) (layers F.Cu B.Cu) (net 10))
 (segment (start 101.15 72.6) (end 100.43 72.6) (width 0.25) (layer F.Cu) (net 10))
 (segment (start 99.75 72.6) (end 100.43 72.6) (width 0.25) (layer F.Cu) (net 10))
 (segment (start 102.2975 83.405) (end 101.985 83.405) (width 0.25) (layer F.Cu) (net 10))
 (via (at 100.54 83.96) (size 0.8) (drill 0.4) (layers F.Cu B.Cu) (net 10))
 (segment (start 101.43 83.96) (end 100.54 83.96) (width 0.25) (layer F.Cu) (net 10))
 (segment (start 101.985 83.405) (end 101.43 83.96) (width 0.25) (layer F.Cu) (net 10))
 (segment (start 100.54 83.96) (end 102.11 83.96) (width 0.25) (layer B.Cu) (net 10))
 (segment (start 102.11 83.96) (end 102.86777 83.20223) (width 0.25) (layer B.Cu) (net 10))
 (segment (start 102.86777 83.20223) (end 102.86777 75.79) (width 0.25) (layer B.Cu) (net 10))
 (segment (start 102.86777 75.79) (end 102.15 75.07223) (width 0.25) (layer B.Cu) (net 10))
 (segment (start 102.15 73.05) (end 101.7 72.6) (width 0.25) (layer B.Cu) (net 10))
 (segment (start 102.15 75.07223) (end 102.15 73.05) (width 0.25) (layer B.Cu) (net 10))
 (segment (start 100.43 72.6) (end 101.7 72.6) (width 0.25) (layer B.Cu) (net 10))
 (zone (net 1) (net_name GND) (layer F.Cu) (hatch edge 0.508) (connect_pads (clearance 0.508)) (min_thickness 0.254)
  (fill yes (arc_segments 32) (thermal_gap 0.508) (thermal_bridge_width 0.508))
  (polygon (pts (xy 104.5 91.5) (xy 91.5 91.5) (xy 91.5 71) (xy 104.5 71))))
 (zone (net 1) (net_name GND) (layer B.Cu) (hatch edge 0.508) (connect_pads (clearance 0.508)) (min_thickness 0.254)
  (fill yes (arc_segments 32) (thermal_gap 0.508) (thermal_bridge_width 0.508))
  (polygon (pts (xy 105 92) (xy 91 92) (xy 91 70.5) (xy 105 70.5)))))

